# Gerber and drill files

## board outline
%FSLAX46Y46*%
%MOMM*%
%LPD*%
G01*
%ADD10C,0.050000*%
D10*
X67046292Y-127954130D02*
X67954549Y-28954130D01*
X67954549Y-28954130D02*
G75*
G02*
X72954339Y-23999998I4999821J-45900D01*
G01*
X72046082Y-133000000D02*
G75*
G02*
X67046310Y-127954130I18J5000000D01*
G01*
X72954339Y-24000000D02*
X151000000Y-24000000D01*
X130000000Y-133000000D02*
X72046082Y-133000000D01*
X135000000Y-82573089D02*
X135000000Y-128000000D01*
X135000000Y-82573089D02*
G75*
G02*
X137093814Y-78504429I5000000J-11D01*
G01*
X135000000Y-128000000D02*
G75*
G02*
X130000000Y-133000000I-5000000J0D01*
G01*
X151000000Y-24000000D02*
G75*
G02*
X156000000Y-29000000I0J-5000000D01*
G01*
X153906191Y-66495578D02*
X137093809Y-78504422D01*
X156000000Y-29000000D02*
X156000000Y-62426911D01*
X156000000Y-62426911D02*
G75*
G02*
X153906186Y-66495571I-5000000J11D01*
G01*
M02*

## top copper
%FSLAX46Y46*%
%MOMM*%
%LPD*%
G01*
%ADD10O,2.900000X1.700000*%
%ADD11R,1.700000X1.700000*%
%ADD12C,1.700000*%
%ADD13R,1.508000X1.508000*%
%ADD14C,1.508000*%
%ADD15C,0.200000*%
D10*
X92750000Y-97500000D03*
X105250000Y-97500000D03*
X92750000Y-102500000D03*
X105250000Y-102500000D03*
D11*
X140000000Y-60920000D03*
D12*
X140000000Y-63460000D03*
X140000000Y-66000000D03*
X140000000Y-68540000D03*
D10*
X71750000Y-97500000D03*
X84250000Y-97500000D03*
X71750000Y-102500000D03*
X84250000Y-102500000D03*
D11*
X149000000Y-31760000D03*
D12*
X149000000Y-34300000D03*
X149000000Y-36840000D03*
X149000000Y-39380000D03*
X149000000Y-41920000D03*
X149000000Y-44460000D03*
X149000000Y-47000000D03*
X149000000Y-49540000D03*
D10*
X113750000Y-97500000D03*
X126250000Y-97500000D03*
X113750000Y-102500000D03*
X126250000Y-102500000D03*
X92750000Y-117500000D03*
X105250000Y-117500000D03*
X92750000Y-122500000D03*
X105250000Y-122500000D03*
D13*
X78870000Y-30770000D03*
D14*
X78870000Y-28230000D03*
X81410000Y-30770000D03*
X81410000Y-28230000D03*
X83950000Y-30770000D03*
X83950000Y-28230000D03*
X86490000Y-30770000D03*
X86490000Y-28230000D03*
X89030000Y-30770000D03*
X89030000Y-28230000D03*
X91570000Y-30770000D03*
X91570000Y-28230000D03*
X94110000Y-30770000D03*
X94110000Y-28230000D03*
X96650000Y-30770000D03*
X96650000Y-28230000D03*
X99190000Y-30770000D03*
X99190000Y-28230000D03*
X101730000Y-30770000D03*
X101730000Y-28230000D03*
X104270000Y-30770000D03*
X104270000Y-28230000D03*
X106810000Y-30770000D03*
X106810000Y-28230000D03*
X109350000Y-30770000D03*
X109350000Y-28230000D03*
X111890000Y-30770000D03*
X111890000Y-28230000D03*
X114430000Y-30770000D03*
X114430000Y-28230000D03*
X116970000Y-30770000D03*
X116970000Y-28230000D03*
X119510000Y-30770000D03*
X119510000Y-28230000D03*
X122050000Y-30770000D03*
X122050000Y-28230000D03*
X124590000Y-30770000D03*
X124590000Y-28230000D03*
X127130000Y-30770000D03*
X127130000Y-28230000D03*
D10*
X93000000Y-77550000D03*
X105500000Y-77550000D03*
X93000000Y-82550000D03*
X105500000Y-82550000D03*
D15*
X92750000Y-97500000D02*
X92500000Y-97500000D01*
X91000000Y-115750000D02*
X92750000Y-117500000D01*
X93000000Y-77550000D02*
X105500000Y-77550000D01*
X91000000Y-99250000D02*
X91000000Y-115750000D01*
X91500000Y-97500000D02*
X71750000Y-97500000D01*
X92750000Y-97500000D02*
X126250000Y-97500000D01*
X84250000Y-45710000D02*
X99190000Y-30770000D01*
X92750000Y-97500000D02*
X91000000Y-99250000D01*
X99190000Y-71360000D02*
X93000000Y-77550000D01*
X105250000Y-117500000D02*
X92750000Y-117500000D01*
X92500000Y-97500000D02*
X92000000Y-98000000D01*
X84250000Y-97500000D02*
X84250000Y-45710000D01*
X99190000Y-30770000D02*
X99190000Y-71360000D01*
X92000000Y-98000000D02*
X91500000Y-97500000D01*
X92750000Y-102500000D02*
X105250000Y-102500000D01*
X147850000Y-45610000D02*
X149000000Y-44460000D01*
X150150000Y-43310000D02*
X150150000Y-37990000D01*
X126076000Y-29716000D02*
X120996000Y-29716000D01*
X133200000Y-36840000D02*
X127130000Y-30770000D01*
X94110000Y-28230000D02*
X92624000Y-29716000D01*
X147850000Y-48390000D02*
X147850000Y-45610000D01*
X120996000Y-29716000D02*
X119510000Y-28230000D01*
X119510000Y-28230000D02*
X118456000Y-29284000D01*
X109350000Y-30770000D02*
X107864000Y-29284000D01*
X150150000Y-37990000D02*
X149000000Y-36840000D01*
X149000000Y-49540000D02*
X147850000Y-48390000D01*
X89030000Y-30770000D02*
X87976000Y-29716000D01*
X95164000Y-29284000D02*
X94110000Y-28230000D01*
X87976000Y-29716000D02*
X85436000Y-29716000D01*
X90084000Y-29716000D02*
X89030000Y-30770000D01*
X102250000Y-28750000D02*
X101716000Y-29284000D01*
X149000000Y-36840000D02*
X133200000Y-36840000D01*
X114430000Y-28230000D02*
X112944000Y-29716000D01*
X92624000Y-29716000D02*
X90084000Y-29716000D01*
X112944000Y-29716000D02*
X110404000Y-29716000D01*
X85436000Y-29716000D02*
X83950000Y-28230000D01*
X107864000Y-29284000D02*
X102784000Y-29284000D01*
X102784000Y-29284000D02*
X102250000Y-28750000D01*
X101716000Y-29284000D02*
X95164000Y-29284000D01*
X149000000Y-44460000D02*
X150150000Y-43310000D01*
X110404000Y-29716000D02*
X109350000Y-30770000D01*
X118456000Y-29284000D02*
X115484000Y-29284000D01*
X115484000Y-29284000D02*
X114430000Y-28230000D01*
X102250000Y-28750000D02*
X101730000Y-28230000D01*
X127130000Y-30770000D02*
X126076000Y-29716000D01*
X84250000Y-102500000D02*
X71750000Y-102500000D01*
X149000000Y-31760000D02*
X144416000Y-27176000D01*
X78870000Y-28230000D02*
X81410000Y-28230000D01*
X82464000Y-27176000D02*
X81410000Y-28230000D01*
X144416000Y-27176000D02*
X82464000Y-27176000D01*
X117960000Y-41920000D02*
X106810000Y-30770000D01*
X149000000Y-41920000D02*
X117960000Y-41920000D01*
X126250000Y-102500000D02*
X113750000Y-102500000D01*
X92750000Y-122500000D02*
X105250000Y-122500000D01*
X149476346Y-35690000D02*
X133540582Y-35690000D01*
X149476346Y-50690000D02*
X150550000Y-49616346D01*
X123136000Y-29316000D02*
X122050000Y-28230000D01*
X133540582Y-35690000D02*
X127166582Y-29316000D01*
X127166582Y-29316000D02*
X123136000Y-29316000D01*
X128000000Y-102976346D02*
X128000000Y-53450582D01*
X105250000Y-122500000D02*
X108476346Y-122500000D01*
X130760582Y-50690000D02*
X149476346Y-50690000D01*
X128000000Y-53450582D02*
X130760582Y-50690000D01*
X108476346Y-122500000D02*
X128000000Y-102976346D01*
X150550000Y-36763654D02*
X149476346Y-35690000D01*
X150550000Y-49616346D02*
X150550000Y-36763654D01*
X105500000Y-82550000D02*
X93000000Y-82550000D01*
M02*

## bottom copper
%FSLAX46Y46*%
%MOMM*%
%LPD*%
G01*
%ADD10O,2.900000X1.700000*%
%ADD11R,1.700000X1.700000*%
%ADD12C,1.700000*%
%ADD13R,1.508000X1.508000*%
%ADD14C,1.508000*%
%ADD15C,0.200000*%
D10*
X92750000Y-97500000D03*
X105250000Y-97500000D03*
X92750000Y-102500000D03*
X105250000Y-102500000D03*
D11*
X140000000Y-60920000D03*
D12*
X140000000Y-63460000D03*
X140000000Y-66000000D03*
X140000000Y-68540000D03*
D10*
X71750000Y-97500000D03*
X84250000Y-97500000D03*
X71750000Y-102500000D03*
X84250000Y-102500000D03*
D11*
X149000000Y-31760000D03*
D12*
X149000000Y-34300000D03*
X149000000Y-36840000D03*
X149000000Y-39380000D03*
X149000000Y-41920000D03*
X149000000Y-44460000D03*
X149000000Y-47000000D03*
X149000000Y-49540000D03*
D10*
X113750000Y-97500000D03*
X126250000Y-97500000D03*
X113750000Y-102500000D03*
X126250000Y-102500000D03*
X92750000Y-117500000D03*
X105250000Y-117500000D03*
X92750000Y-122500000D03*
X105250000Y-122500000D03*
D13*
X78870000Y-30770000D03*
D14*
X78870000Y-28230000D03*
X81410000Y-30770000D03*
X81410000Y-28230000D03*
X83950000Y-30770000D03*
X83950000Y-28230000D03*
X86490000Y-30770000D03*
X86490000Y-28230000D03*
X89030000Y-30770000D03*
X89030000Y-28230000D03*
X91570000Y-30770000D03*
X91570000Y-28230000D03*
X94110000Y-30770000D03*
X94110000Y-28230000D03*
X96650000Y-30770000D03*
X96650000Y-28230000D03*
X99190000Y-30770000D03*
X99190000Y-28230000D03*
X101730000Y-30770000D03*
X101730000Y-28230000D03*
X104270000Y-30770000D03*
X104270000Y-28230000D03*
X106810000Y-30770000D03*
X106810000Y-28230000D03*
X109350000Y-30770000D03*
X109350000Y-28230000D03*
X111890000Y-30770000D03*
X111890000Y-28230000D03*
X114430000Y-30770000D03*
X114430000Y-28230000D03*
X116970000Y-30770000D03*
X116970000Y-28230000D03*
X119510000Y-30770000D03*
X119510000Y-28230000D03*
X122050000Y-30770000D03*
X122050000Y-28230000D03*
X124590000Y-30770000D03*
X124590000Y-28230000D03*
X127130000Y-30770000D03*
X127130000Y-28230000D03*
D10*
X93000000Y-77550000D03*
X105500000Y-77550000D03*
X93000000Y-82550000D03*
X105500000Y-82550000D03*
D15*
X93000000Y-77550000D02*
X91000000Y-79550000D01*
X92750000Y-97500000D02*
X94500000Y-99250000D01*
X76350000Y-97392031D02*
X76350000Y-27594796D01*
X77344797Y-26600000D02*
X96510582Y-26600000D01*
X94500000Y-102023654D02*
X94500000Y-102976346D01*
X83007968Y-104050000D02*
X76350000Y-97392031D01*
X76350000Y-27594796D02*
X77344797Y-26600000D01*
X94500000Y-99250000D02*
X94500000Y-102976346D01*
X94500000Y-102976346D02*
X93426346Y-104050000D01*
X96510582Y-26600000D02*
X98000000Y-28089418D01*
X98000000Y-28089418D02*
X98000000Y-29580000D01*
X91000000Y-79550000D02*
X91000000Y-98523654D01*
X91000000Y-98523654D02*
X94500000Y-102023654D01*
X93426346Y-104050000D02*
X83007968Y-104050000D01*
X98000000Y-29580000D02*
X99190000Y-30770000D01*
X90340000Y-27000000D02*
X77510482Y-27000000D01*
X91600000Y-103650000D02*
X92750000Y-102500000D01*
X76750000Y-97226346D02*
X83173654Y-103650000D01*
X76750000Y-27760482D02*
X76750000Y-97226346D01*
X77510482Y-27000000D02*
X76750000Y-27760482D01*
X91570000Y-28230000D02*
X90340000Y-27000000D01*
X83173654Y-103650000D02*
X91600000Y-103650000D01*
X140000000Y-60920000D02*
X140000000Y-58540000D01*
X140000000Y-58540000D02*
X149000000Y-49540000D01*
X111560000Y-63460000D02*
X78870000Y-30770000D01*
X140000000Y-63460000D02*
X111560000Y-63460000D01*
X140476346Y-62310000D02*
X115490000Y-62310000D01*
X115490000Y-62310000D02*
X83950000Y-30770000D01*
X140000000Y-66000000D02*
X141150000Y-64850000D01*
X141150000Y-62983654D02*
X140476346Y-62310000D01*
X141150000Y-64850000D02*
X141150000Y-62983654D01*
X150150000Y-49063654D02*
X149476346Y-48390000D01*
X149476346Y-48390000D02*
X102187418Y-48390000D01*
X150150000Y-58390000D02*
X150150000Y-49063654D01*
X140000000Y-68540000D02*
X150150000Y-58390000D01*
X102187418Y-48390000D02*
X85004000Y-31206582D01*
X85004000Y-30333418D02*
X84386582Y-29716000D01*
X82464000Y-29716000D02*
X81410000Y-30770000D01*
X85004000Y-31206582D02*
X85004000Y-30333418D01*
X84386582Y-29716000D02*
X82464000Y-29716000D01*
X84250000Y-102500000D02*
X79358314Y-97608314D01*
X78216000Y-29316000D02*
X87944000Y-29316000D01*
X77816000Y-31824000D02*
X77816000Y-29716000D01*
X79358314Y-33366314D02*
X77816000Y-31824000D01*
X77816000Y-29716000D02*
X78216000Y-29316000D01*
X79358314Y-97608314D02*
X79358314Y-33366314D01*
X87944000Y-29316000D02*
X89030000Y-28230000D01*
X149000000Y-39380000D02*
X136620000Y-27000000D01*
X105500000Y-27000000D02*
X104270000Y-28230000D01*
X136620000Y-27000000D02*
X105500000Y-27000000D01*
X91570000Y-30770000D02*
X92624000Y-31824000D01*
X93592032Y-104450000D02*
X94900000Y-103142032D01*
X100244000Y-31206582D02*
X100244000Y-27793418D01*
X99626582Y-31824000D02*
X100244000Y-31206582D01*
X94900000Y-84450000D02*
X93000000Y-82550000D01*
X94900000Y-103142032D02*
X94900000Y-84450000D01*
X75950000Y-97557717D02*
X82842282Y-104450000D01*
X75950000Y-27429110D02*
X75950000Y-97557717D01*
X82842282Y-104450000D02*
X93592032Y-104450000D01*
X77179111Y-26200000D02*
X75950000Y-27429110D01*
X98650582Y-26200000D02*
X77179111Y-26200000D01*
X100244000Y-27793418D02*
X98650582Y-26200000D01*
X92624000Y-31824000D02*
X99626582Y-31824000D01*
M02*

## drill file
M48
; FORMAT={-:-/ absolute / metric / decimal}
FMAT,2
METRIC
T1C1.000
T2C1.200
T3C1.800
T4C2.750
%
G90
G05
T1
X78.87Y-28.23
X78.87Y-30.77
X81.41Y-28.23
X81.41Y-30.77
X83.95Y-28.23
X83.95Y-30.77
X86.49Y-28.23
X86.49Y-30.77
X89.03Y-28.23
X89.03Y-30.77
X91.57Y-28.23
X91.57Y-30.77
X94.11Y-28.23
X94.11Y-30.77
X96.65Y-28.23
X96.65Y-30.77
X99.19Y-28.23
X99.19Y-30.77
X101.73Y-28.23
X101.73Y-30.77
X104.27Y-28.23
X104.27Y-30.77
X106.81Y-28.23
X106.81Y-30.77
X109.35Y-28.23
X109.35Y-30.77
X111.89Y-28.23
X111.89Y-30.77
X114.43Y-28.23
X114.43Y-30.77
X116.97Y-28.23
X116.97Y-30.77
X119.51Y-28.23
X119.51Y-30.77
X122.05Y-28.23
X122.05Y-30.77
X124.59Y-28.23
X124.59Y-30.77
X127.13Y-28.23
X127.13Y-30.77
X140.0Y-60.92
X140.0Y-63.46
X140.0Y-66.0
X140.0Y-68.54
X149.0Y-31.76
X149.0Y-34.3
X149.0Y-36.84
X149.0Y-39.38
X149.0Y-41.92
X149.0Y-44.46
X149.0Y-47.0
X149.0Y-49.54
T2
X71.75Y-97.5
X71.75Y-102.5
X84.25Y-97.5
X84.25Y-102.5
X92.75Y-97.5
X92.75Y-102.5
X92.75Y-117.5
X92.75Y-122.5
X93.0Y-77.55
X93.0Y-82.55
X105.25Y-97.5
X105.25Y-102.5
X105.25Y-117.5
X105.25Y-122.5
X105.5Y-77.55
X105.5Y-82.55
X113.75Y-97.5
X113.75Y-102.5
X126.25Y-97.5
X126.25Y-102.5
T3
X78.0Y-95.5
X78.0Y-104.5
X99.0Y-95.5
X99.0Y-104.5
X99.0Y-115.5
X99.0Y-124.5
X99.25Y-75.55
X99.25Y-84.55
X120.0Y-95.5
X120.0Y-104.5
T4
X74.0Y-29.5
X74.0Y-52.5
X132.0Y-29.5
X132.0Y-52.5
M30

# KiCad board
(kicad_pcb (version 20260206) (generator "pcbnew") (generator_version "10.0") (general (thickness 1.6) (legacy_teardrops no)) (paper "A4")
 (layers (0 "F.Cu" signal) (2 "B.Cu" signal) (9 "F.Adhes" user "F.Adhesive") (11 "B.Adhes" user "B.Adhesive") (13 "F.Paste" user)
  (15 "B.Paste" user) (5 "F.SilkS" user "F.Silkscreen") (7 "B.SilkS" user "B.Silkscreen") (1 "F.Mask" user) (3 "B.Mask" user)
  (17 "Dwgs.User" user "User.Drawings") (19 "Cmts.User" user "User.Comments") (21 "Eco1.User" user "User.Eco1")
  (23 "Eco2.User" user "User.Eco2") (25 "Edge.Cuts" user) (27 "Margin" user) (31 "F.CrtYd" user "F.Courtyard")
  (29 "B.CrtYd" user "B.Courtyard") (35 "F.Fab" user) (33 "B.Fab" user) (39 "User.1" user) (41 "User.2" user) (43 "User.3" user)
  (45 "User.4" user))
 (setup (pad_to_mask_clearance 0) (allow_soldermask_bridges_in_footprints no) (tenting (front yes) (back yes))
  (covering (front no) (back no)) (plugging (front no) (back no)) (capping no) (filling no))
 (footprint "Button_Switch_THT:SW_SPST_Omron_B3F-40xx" (layer "F.Cu") (at 92.75 97.5)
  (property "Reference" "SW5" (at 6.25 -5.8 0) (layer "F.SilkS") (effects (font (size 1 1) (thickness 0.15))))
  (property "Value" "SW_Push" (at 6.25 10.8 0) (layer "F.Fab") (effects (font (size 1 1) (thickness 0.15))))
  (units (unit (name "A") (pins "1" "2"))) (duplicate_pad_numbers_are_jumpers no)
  (pad "" np_thru_hole circle (at 6.25 -2) (size 1.8 1.8) (drill 1.8) (layers "*.Cu" "*.Mask"))
  (pad "" np_thru_hole circle (at 6.25 7) (size 1.8 1.8) (drill 1.8) (layers "*.Cu" "*.Mask"))
  (pad "1" thru_hole oval (at 0 0) (size 2.9 1.7) (drill 1.2) (layers "*.Cu" "*.Mask") (remove_unused_layers no) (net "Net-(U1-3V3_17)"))
  (pad "1" thru_hole oval (at 12.5 0) (size 2.9 1.7) (drill 1.2) (layers "*.Cu" "*.Mask") (remove_unused_layers no) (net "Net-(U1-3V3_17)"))
  (pad "2" thru_hole oval (at 0 5) (size 2.9 1.7) (drill 1.2) (layers "*.Cu" "*.Mask") (remove_unused_layers no)
   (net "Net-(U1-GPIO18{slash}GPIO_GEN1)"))
  (pad "2" thru_hole oval (at 12.5 5) (size 2.9 1.7) (drill 1.2) (layers "*.Cu" "*.Mask") (remove_unused_layers no)
   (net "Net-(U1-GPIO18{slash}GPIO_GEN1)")))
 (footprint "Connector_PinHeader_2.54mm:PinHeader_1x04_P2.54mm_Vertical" (layer "F.Cu") (at 140 60.92)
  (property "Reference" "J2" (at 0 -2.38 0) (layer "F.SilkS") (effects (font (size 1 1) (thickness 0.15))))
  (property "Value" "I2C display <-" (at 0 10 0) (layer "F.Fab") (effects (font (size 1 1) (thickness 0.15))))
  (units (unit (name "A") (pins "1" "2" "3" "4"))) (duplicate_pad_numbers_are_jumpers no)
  (pad "1" thru_hole rect (at 0 0) (size 1.7 1.7) (drill 1) (layers "*.Cu" "*.Mask") (remove_unused_layers no) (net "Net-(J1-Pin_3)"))
  (pad "2" thru_hole circle (at 0 2.54) (size 1.7 1.7) (drill 1) (layers "*.Cu" "*.Mask") (remove_unused_layers no) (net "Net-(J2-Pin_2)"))
  (pad "3" thru_hole circle (at 0 5.08) (size 1.7 1.7) (drill 1) (layers "*.Cu" "*.Mask") (remove_unused_layers no) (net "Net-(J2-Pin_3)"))
  (pad "4" thru_hole circle (at 0 7.62) (size 1.7 1.7) (drill 1) (layers "*.Cu" "*.Mask") (remove_unused_layers no) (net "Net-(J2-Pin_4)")))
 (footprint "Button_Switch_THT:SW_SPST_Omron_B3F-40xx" (layer "F.Cu") (at 71.75 97.5)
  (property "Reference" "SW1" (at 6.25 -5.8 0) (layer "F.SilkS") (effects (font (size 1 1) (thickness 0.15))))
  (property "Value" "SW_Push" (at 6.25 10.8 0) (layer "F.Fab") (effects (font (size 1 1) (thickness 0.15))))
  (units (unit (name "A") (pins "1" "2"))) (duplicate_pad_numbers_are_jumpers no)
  (pad "" np_thru_hole circle (at 6.25 -2) (size 1.8 1.8) (drill 1.8) (layers "*.Cu" "*.Mask"))
  (pad "" np_thru_hole circle (at 6.25 7) (size 1.8 1.8) (drill 1.8) (layers "*.Cu" "*.Mask"))
  (pad "1" thru_hole oval (at 0 0) (size 2.9 1.7) (drill 1.2) (layers "*.Cu" "*.Mask") (remove_unused_layers no) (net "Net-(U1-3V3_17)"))
  (pad "1" thru_hole oval (at 12.5 0) (size 2.9 1.7) (drill 1.2) (layers "*.Cu" "*.Mask") (remove_unused_layers no) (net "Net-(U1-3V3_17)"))
  (pad "2" thru_hole oval (at 0 5) (size 2.9 1.7) (drill 1.2) (layers "*.Cu" "*.Mask") (remove_unused_layers no)
   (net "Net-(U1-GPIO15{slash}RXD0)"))
  (pad "2" thru_hole oval (at 12.5 5) (size 2.9 1.7) (drill 1.2) (layers "*.Cu" "*.Mask") (remove_unused_layers no)
   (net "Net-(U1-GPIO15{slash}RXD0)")))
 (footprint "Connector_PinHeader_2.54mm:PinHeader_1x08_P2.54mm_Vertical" (layer "F.Cu") (at 149 31.76)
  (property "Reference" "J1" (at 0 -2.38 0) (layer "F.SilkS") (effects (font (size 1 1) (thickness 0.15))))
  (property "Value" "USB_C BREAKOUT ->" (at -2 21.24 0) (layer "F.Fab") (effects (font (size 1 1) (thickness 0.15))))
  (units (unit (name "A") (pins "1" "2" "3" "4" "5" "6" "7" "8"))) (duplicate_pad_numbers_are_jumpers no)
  (pad "1" thru_hole rect (at 0 0) (size 1.7 1.7) (drill 1) (layers "*.Cu" "*.Mask") (remove_unused_layers no) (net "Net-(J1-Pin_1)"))
  (pad "2" thru_hole circle (at 0 2.54) (size 1.7 1.7) (drill 1) (layers "*.Cu" "*.Mask") (remove_unused_layers no)
   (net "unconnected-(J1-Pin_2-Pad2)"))
  (pad "3" thru_hole circle (at 0 5.08) (size 1.7 1.7) (drill 1) (layers "*.Cu" "*.Mask") (remove_unused_layers no) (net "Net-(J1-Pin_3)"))
  (pad "4" thru_hole circle (at 0 7.62) (size 1.7 1.7) (drill 1) (layers "*.Cu" "*.Mask") (remove_unused_layers no) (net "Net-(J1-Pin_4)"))
  (pad "5" thru_hole circle (at 0 10.16) (size 1.7 1.7) (drill 1) (layers "*.Cu" "*.Mask") (remove_unused_layers no) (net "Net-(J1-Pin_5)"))
  (pad "6" thru_hole circle (at 0 12.7) (size 1.7 1.7) (drill 1) (layers "*.Cu" "*.Mask") (remove_unused_layers no) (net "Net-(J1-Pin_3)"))
  (pad "7" thru_hole circle (at 0 15.24) (size 1.7 1.7) (drill 1) (layers "*.Cu" "*.Mask") (remove_unused_layers no)
   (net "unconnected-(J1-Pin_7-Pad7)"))
  (pad "8" thru_hole circle (at 0 17.78) (size 1.7 1.7) (drill 1) (layers "*.Cu" "*.Mask") (remove_unused_layers no) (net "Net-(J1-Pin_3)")))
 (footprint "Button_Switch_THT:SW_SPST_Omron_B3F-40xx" (layer "F.Cu") (at 113.75 97.5)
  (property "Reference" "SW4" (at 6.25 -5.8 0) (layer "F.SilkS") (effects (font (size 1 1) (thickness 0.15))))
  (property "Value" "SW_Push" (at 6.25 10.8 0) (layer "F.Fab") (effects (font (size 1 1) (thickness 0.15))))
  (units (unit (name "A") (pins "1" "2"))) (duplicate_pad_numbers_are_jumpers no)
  (pad "" np_thru_hole circle (at 6.25 -2) (size 1.8 1.8) (drill 1.8) (layers "*.Cu" "*.Mask"))
  (pad "" np_thru_hole circle (at 6.25 7) (size 1.8 1.8) (drill 1.8) (layers "*.Cu" "*.Mask"))
  (pad "1" thru_hole oval (at 0 0) (size 2.9 1.7) (drill 1.2) (layers "*.Cu" "*.Mask") (remove_unused_layers no) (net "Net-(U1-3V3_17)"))
  (pad "1" thru_hole oval (at 12.5 0) (size 2.9 1.7) (drill 1.2) (layers "*.Cu" "*.Mask") (remove_unused_layers no) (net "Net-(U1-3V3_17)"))
  (pad "2" thru_hole oval (at 0 5) (size 2.9 1.7) (drill 1.2) (layers "*.Cu" "*.Mask") (remove_unused_layers no)
   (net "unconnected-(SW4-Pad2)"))
  (pad "2" thru_hole oval (at 12.5 5) (size 2.9 1.7) (drill 1.2) (layers "*.Cu" "*.Mask") (remove_unused_layers no)
   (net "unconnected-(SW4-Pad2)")))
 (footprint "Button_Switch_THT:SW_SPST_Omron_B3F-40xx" (layer "F.Cu") (at 92.75 117.5)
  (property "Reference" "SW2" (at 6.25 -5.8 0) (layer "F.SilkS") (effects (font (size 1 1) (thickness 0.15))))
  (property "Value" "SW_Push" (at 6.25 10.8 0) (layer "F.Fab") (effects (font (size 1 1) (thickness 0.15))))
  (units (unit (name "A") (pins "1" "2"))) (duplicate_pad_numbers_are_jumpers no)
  (pad "" np_thru_hole circle (at 6.25 -2) (size 1.8 1.8) (drill 1.8) (layers "*.Cu" "*.Mask"))
  (pad "" np_thru_hole circle (at 6.25 7) (size 1.8 1.8) (drill 1.8) (layers "*.Cu" "*.Mask"))
  (pad "1" thru_hole oval (at 0 0) (size 2.9 1.7) (drill 1.2) (layers "*.Cu" "*.Mask") (remove_unused_layers no) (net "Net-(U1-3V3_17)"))
  (pad "1" thru_hole oval (at 12.5 0) (size 2.9 1.7) (drill 1.2) (layers "*.Cu" "*.Mask") (remove_unused_layers no) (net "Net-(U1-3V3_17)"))
  (pad "2" thru_hole oval (at 0 5) (size 2.9 1.7) (drill 1.2) (layers "*.Cu" "*.Mask") (remove_unused_layers no) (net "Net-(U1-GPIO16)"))
  (pad "2" thru_hole oval (at 12.5 5) (size 2.9 1.7) (drill 1.2) (layers "*.Cu" "*.Mask") (remove_unused_layers no) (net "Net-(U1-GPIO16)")))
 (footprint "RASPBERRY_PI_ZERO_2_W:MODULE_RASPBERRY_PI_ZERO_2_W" (layer "F.Cu") (at 103 41)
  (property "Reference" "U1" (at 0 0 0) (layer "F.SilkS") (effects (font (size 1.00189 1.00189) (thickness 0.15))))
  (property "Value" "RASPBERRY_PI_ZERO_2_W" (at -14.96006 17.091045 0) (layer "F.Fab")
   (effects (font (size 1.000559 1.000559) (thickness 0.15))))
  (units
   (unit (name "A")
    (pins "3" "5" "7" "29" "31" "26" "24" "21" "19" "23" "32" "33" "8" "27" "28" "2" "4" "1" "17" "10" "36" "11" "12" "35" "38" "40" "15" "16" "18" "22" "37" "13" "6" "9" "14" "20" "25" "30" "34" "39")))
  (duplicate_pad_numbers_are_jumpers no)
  (pad "" np_thru_hole circle (at -29 -11.5) (size 2.75 2.75) (drill 2.75) (layers "*.Cu" "*.Mask"))
  (pad "" np_thru_hole circle (at -29 11.5) (size 2.75 2.75) (drill 2.75) (layers "*.Cu" "*.Mask"))
  (pad "" np_thru_hole circle (at 29 -11.5) (size 2.75 2.75) (drill 2.75) (layers "*.Cu" "*.Mask"))
  (pad "" np_thru_hole circle (at 29 11.5) (size 2.75 2.75) (drill 2.75) (layers "*.Cu" "*.Mask"))
  (pad "1" thru_hole rect (at -24.13 -10.23) (size 1.508 1.508) (drill 1) (layers "*.Cu" "*.Mask") (remove_unused_layers no)
   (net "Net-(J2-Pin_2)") (solder_mask_margin 0.102))
  (pad "2" thru_hole circle (at -24.13 -12.77) (size 1.508 1.508) (drill 1) (layers "*.Cu" "*.Mask") (remove_unused_layers no)
   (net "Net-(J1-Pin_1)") (solder_mask_margin 0.102))
  (pad "3" thru_hole circle (at -21.59 -10.23) (size 1.508 1.508) (drill 1) (layers "*.Cu" "*.Mask") (remove_unused_layers no)
   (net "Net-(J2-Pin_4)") (solder_mask_margin 0.102))
  (pad "4" thru_hole circle (at -21.59 -12.77) (size 1.508 1.508) (drill 1) (layers "*.Cu" "*.Mask") (remove_unused_layers no)
   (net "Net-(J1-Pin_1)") (solder_mask_margin 0.102))
  (pad "5" thru_hole circle (at -19.05 -10.23) (size 1.508 1.508) (drill 1) (layers "*.Cu" "*.Mask") (remove_unused_layers no)
   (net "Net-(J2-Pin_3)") (solder_mask_margin 0.102))
  (pad "6" thru_hole circle (at -19.05 -12.77) (size 1.508 1.508) (drill 1) (layers "*.Cu" "*.Mask") (remove_unused_layers no)
   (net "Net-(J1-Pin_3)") (solder_mask_margin 0.102))
  (pad "7" thru_hole circle (at -16.51 -10.23) (size 1.508 1.508) (drill 1) (layers "*.Cu" "*.Mask") (remove_unused_layers no)
   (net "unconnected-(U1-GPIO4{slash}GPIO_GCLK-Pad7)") (solder_mask_margin 0.102))
  (pad "8" thru_hole circle (at -16.51 -12.77) (size 1.508 1.508) (drill 1) (layers "*.Cu" "*.Mask") (remove_unused_layers no)
   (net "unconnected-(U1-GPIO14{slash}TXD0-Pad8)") (solder_mask_margin 0.102))
  (pad "9" thru_hole circle (at -13.97 -10.23) (size 1.508 1.508) (drill 1) (layers "*.Cu" "*.Mask") (remove_unused_layers no)
   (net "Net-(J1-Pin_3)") (solder_mask_margin 0.102))
  (pad "10" thru_hole circle (at -13.97 -12.77) (size 1.508 1.508) (drill 1) (layers "*.Cu" "*.Mask") (remove_unused_layers no)
   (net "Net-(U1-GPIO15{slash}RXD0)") (solder_mask_margin 0.102))
  (pad "11" thru_hole circle (at -11.43 -10.23) (size 1.508 1.508) (drill 1) (layers "*.Cu" "*.Mask") (remove_unused_layers no)
   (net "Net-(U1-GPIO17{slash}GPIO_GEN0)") (solder_mask_margin 0.102))
  (pad "12" thru_hole circle (at -11.43 -12.77) (size 1.508 1.508) (drill 1) (layers "*.Cu" "*.Mask") (remove_unused_layers no)
   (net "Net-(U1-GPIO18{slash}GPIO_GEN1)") (solder_mask_margin 0.102))
  (pad "13" thru_hole circle (at -8.89 -10.23) (size 1.508 1.508) (drill 1) (layers "*.Cu" "*.Mask") (remove_unused_layers no)
   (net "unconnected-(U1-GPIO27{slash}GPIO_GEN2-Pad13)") (solder_mask_margin 0.102))
  (pad "14" thru_hole circle (at -8.89 -12.77) (size 1.508 1.508) (drill 1) (layers "*.Cu" "*.Mask") (remove_unused_layers no)
   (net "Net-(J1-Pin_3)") (solder_mask_margin 0.102))
  (pad "15" thru_hole circle (at -6.35 -10.23) (size 1.508 1.508) (drill 1) (layers "*.Cu" "*.Mask") (remove_unused_layers no)
   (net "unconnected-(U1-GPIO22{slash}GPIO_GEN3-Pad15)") (solder_mask_margin 0.102))
  (pad "16" thru_hole circle (at -6.35 -12.77) (size 1.508 1.508) (drill 1) (layers "*.Cu" "*.Mask") (remove_unused_layers no)
   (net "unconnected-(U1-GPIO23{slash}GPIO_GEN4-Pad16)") (solder_mask_margin 0.102))
  (pad "17" thru_hole circle (at -3.81 -10.23) (size 1.508 1.508) (drill 1) (layers "*.Cu" "*.Mask") (remove_unused_layers no)
   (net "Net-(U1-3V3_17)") (solder_mask_margin 0.102))
  (pad "18" thru_hole circle (at -3.81 -12.77) (size 1.508 1.508) (drill 1) (layers "*.Cu" "*.Mask") (remove_unused_layers no)
   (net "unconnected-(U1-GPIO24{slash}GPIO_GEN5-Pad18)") (solder_mask_margin 0.102))
  (pad "19" thru_hole circle (at -1.27 -10.23) (size 1.508 1.508) (drill 1) (layers "*.Cu" "*.Mask") (remove_unused_layers no)
   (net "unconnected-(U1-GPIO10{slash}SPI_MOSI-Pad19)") (solder_mask_margin 0.102))
  (pad "20" thru_hole circle (at -1.27 -12.77) (size 1.508 1.508) (drill 1) (layers "*.Cu" "*.Mask") (remove_unused_layers no)
   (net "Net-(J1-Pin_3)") (solder_mask_margin 0.102))
  (pad "21" thru_hole circle (at 1.27 -10.23) (size 1.508 1.508) (drill 1) (layers "*.Cu" "*.Mask") (remove_unused_layers no)
   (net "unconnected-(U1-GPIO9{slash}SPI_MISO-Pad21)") (solder_mask_margin 0.102))
  (pad "22" thru_hole circle (at 1.27 -12.77) (size 1.508 1.508) (drill 1) (layers "*.Cu" "*.Mask") (remove_unused_layers no)
   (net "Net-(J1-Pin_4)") (solder_mask_margin 0.102))
  (pad "23" thru_hole circle (at 3.81 -10.23) (size 1.508 1.508) (drill 1) (layers "*.Cu" "*.Mask") (remove_unused_layers no)
   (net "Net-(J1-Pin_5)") (solder_mask_margin 0.102))
  (pad "24" thru_hole circle (at 3.81 -12.77) (size 1.508 1.508) (drill 1) (layers "*.Cu" "*.Mask") (remove_unused_layers no)
   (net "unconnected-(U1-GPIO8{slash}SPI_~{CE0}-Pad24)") (solder_mask_margin 0.102))
  (pad "25" thru_hole circle (at 6.35 -10.23) (size 1.508 1.508) (drill 1) (layers "*.Cu" "*.Mask") (remove_unused_layers no)
   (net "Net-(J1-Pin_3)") (solder_mask_margin 0.102))
  (pad "26" thru_hole circle (at 6.35 -12.77) (size 1.508 1.508) (drill 1) (layers "*.Cu" "*.Mask") (remove_unused_layers no)
   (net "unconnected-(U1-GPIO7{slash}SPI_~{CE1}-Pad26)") (solder_mask_margin 0.102))
  (pad "27" thru_hole circle (at 8.89 -10.23) (size 1.508 1.508) (drill 1) (layers "*.Cu" "*.Mask") (remove_unused_layers no)
   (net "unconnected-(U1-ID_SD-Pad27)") (solder_mask_margin 0.102))
  (pad "28" thru_hole circle (at 8.89 -12.77) (size 1.508 1.508) (drill 1) (layers "*.Cu" "*.Mask") (remove_unused_layers no)
   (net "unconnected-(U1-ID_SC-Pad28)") (solder_mask_margin 0.102))
  (pad "29" thru_hole circle (at 11.43 -10.23) (size 1.508 1.508) (drill 1) (layers "*.Cu" "*.Mask") (remove_unused_layers no)
   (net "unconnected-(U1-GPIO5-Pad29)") (solder_mask_margin 0.102))
  (pad "30" thru_hole circle (at 11.43 -12.77) (size 1.508 1.508) (drill 1) (layers "*.Cu" "*.Mask") (remove_unused_layers no)
   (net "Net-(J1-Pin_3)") (solder_mask_margin 0.102))
  (pad "31" thru_hole circle (at 13.97 -10.23) (size 1.508 1.508) (drill 1) (layers "*.Cu" "*.Mask") (remove_unused_layers no)
   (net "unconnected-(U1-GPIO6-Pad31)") (solder_mask_margin 0.102))
  (pad "32" thru_hole circle (at 13.97 -12.77) (size 1.508 1.508) (drill 1) (layers "*.Cu" "*.Mask") (remove_unused_layers no)
   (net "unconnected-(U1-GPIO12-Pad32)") (solder_mask_margin 0.102))
  (pad "33" thru_hole circle (at 16.51 -10.23) (size 1.508 1.508) (drill 1) (layers "*.Cu" "*.Mask") (remove_unused_layers no)
   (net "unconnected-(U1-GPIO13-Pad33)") (solder_mask_margin 0.102))
  (pad "34" thru_hole circle (at 16.51 -12.77) (size 1.508 1.508) (drill 1) (layers "*.Cu" "*.Mask") (remove_unused_layers no)
   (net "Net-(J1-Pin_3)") (solder_mask_margin 0.102))
  (pad "35" thru_hole circle (at 19.05 -10.23) (size 1.508 1.508) (drill 1) (layers "*.Cu" "*.Mask") (remove_unused_layers no)
   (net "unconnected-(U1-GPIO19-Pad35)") (solder_mask_margin 0.102))
  (pad "36" thru_hole circle (at 19.05 -12.77) (size 1.508 1.508) (drill 1) (layers "*.Cu" "*.Mask") (remove_unused_layers no)
   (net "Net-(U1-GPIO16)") (solder_mask_margin 0.102))
  (pad "37" thru_hole circle (at 21.59 -10.23) (size 1.508 1.508) (drill 1) (layers "*.Cu" "*.Mask") (remove_unused_layers no)
   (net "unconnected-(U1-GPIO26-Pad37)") (solder_mask_margin 0.102))
  (pad "38" thru_hole circle (at 21.59 -12.77) (size 1.508 1.508) (drill 1) (layers "*.Cu" "*.Mask") (remove_unused_layers no)
   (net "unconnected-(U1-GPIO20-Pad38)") (solder_mask_margin 0.102))
  (pad "39" thru_hole circle (at 24.13 -10.23) (size 1.508 1.508) (drill 1) (layers "*.Cu" "*.Mask") (remove_unused_layers no)
   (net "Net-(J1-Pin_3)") (solder_mask_margin 0.102))
  (pad "40" thru_hole circle (at 24.13 -12.77) (size 1.508 1.508) (drill 1) (layers "*.Cu" "*.Mask") (remove_unused_layers no)
   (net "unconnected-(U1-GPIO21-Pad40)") (solder_mask_margin 0.102)))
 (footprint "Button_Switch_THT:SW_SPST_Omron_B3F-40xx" (layer "F.Cu") (at 93 77.55)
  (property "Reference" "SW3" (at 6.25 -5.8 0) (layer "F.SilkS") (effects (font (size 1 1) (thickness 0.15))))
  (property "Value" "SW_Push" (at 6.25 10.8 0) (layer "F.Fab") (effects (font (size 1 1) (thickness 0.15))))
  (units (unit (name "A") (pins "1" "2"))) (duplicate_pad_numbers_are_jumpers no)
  (pad "" np_thru_hole circle (at 6.25 -2) (size 1.8 1.8) (drill 1.8) (layers "*.Cu" "*.Mask"))
  (pad "" np_thru_hole circle (at 6.25 7) (size 1.8 1.8) (drill 1.8) (layers "*.Cu" "*.Mask"))
  (pad "1" thru_hole oval (at 0 0) (size 2.9 1.7) (drill 1.2) (layers "*.Cu" "*.Mask") (remove_unused_layers no) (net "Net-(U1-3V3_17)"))
  (pad "1" thru_hole oval (at 12.5 0) (size 2.9 1.7) (drill 1.2) (layers "*.Cu" "*.Mask") (remove_unused_layers no) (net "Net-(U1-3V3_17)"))
  (pad "2" thru_hole oval (at 0 5) (size 2.9 1.7) (drill 1.2) (layers "*.Cu" "*.Mask") (remove_unused_layers no)
   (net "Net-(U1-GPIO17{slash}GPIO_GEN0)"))
  (pad "2" thru_hole oval (at 12.5 5) (size 2.9 1.7) (drill 1.2) (layers "*.Cu" "*.Mask") (remove_unused_layers no)
   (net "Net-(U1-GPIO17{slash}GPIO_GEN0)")))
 (gr_line (start 67.046292 127.95413) (end 67.954549 28.95413) (stroke (width 0.05) (type default)) (layer "Edge.Cuts"))
 (gr_arc (start 67.954549 28.95413) (mid 69.435062 25.448299) (end 72.954339 24) (stroke (width 0.05) (type default)) (layer "Edge.Cuts"))
 (gr_arc (start 72.046082 133) (mid 68.494368 131.519279) (end 67.046292 127.95413) (stroke (width 0.05) (type default)) (layer "Edge.Cuts"))
 (gr_line (start 72.954339 24) (end 151 24) (stroke (width 0.05) (type default)) (layer "Edge.Cuts"))
 (gr_line (start 130 133) (end 72.046082 133) (stroke (width 0.05) (type default)) (layer "Edge.Cuts"))
 (gr_line (start 135 82.573089) (end 135 128) (stroke (width 0.05) (type default)) (layer "Edge.Cuts"))
 (gr_arc (start 135 82.573089) (mid 135.554166 80.285184) (end 137.093809 78.504422) (stroke (width 0.05) (type default))
  (layer "Edge.Cuts"))
 (gr_arc (start 135 128) (mid 133.535534 131.535534) (end 130 133) (stroke (width 0.05) (type default)) (layer "Edge.Cuts"))
 (gr_arc (start 151 24) (mid 154.535534 25.464466) (end 156 29) (stroke (width 0.05) (type default)) (layer "Edge.Cuts"))
 (gr_line (start 153.906191 66.495578) (end 137.093809 78.504422) (stroke (width 0.05) (type default)) (layer "Edge.Cuts"))
 (gr_line (start 156 29) (end 156 62.426911) (stroke (width 0.05) (type default)) (layer "Edge.Cuts"))
 (gr_arc (start 156 62.426911) (mid 155.445834 64.714816) (end 153.906191 66.495578) (stroke (width 0.05) (type default))
  (layer "Edge.Cuts"))
 (segment (start 92.75 97.5) (end 92.5 97.5) (width 0.2) (layer "F.Cu") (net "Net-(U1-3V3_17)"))
 (segment (start 91 115.75) (end 92.75 117.5) (width 0.2) (layer "F.Cu") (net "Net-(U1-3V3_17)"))
 (segment (start 93 77.55) (end 105.5 77.55) (width 0.2) (layer "F.Cu") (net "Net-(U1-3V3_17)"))
 (segment (start 91 99.25) (end 91 115.75) (width 0.2) (layer "F.Cu") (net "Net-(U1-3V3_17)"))
 (segment (start 91.5 97.5) (end 71.75 97.5) (width 0.2) (layer "F.Cu") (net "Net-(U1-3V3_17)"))
 (segment (start 92.75 97.5) (end 126.25 97.5) (width 0.2) (layer "F.Cu") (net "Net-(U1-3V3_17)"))
 (segment (start 84.25 45.71) (end 99.19 30.77) (width 0.2) (layer "F.Cu") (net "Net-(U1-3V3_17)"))
 (segment (start 92.75 97.5) (end 91 99.25) (width 0.2) (layer "F.Cu") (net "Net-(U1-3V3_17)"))
 (segment (start 99.19 71.36) (end 93 77.55) (width 0.2) (layer "F.Cu") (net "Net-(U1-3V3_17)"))
 (segment (start 105.25 117.5) (end 92.75 117.5) (width 0.2) (layer "F.Cu") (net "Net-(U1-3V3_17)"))
 (segment (start 92.5 97.5) (end 92 98) (width 0.2) (layer "F.Cu") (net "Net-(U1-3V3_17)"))
 (segment (start 84.25 97.5) (end 84.25 45.71) (width 0.2) (layer "F.Cu") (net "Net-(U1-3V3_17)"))
 (segment (start 99.19 30.77) (end 99.19 71.36) (width 0.2) (layer "F.Cu") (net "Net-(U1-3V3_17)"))
 (segment (start 92 98) (end 91.5 97.5) (width 0.2) (layer "F.Cu") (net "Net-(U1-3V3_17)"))
 (segment (start 93 77.55) (end 91 79.55) (width 0.2) (layer "B.Cu") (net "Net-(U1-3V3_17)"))
 (segment (start 92.75 97.5) (end 94.5 99.25) (width 0.2) (layer "B.Cu") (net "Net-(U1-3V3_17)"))
 (segment (start 76.35 97.392031) (end 76.35 27.594796) (width 0.2) (layer "B.Cu") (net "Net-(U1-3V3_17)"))
 (segment (start 77.344797 26.6) (end 96.510582 26.6) (width 0.2) (layer "B.Cu") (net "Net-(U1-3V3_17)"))
 (segment (start 94.5 102.023654) (end 94.5 102.976346) (width 0.2) (layer "B.Cu") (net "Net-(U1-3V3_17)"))
 (segment (start 83.007968 104.05) (end 76.35 97.392031) (width 0.2) (layer "B.Cu") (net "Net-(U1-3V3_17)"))
 (segment (start 76.35 27.594796) (end 77.344797 26.6) (width 0.2) (layer "B.Cu") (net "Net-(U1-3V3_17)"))
 (segment (start 94.5 99.25) (end 94.5 102.976346) (width 0.2) (layer "B.Cu") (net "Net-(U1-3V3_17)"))
 (segment (start 94.5 102.976346) (end 93.426346 104.05) (width 0.2) (layer "B.Cu") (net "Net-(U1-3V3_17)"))
 (segment (start 96.510582 26.6) (end 98 28.089418) (width 0.2) (layer "B.Cu") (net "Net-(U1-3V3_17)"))
 (segment (start 98 28.089418) (end 98 29.58) (width 0.2) (layer "B.Cu") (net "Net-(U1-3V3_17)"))
 (segment (start 91 79.55) (end 91 98.523654) (width 0.2) (layer "B.Cu") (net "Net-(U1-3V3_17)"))
 (segment (start 91 98.523654) (end 94.5 102.023654) (width 0.2) (layer "B.Cu") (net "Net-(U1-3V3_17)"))
 (segment (start 93.426346 104.05) (end 83.007968 104.05) (width 0.2) (layer "B.Cu") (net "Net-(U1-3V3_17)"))
 (segment (start 98 29.58) (end 99.19 30.77) (width 0.2) (layer "B.Cu") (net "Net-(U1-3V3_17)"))
 (segment (start 92.75 102.5) (end 105.25 102.5) (width 0.2) (layer "F.Cu") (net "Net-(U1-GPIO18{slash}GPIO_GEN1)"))
 (segment (start 90.34 27) (end 77.510482 27) (width 0.2) (layer "B.Cu") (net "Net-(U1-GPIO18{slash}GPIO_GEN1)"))
 (segment (start 91.6 103.65) (end 92.75 102.5) (width 0.2) (layer "B.Cu") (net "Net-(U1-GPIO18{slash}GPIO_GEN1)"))
 (segment (start 76.75 97.226346) (end 83.173654 103.65) (width 0.2) (layer "B.Cu") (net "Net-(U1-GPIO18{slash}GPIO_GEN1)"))
 (segment (start 76.75 27.760482) (end 76.75 97.226346) (width 0.2) (layer "B.Cu") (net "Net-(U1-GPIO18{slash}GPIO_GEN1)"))
 (segment (start 77.510482 27) (end 76.75 27.760482) (width 0.2) (layer "B.Cu") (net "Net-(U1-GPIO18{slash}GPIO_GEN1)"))
 (segment (start 91.57 28.23) (end 90.34 27) (width 0.2) (layer "B.Cu") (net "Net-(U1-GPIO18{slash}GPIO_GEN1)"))
 (segment (start 83.173654 103.65) (end 91.6 103.65) (width 0.2) (layer "B.Cu") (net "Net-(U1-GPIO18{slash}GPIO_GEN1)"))
 (segment (start 147.85 45.61) (end 149 44.46) (width 0.2) (layer "F.Cu") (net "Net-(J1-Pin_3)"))
 (segment (start 150.15 43.31) (end 150.15 37.99) (width 0.2) (layer "F.Cu") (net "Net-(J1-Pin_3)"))
 (segment (start 126.076 29.716) (end 120.996 29.716) (width 0.2) (layer "F.Cu") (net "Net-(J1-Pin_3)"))
 (segment (start 133.2 36.84) (end 127.13 30.77) (width 0.2) (layer "F.Cu") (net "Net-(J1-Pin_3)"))
 (segment (start 94.11 28.23) (end 92.624 29.716) (width 0.2) (layer "F.Cu") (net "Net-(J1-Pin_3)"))
 (segment (start 147.85 48.39) (end 147.85 45.61) (width 0.2) (layer "F.Cu") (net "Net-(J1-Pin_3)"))
 (segment (start 120.996 29.716) (end 119.51 28.23) (width 0.2) (layer "F.Cu") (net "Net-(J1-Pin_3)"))
 (segment (start 119.51 28.23) (end 118.456 29.284) (width 0.2) (layer "F.Cu") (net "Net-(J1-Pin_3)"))
 (segment (start 109.35 30.77) (end 107.864 29.284) (width 0.2) (layer "F.Cu") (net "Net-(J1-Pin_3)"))
 (segment (start 150.15 37.99) (end 149 36.84) (width 0.2) (layer "F.Cu") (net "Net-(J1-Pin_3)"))
 (segment (start 149 49.54) (end 147.85 48.39) (width 0.2) (layer "F.Cu") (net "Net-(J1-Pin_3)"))
 (segment (start 89.03 30.77) (end 87.976 29.716) (width 0.2) (layer "F.Cu") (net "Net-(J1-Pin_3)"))
 (segment (start 95.164 29.284) (end 94.11 28.23) (width 0.2) (layer "F.Cu") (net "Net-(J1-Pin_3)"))
 (segment (start 87.976 29.716) (end 85.436 29.716) (width 0.2) (layer "F.Cu") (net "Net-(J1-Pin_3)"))
 (segment (start 90.084 29.716) (end 89.03 30.77) (width 0.2) (layer "F.Cu") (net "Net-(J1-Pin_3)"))
 (segment (start 102.25 28.75) (end 101.716 29.284) (width 0.2) (layer "F.Cu") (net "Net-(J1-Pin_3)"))
 (segment (start 149 36.84) (end 133.2 36.84) (width 0.2) (layer "F.Cu") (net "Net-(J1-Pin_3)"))
 (segment (start 114.43 28.23) (end 112.944 29.716) (width 0.2) (layer "F.Cu") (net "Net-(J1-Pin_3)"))
 (segment (start 92.624 29.716) (end 90.084 29.716) (width 0.2) (layer "F.Cu") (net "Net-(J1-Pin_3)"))
 (segment (start 112.944 29.716) (end 110.404 29.716) (width 0.2) (layer "F.Cu") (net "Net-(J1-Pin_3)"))
 (segment (start 85.436 29.716) (end 83.95 28.23) (width 0.2) (layer "F.Cu") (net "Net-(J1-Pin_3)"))
 (segment (start 107.864 29.284) (end 102.784 29.284) (width 0.2) (layer "F.Cu") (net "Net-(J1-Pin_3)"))
 (segment (start 102.784 29.284) (end 102.25 28.75) (width 0.2) (layer "F.Cu") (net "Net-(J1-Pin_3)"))
 (segment (start 101.716 29.284) (end 95.164 29.284) (width 0.2) (layer "F.Cu") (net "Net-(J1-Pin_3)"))
 (segment (start 149 44.46) (end 150.15 43.31) (width 0.2) (layer "F.Cu") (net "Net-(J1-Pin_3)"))
 (segment (start 110.404 29.716) (end 109.35 30.77) (width 0.2) (layer "F.Cu") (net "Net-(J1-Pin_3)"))
 (segment (start 118.456 29.284) (end 115.484 29.284) (width 0.2) (layer "F.Cu") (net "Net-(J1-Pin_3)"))
 (segment (start 115.484 29.284) (end 114.43 28.23) (width 0.2) (layer "F.Cu") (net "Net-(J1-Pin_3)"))
 (segment (start 102.25 28.75) (end 101.73 28.23) (width 0.2) (layer "F.Cu") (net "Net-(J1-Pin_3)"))
 (segment (start 127.13 30.77) (end 126.076 29.716) (width 0.2) (layer "F.Cu") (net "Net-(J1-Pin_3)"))
 (segment (start 140 60.92) (end 140 58.54) (width 0.2) (layer "B.Cu") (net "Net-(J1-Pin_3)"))
 (segment (start 140 58.54) (end 149 49.54) (width 0.2) (layer "B.Cu") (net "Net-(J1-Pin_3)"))
 (segment (start 111.56 63.46) (end 78.87 30.77) (width 0.2) (layer "B.Cu") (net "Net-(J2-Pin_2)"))
 (segment (start 140 63.46) (end 111.56 63.46) (width 0.2) (layer "B.Cu") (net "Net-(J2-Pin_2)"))
 (segment (start 140.476346 62.31) (end 115.49 62.31) (width 0.2) (layer "B.Cu") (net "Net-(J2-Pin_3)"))
 (segment (start 115.49 62.31) (end 83.95 30.77) (width 0.2) (layer "B.Cu") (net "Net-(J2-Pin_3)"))
 (segment (start 140 66) (end 141.15 64.85) (width 0.2) (layer "B.Cu") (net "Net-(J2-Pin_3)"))
 (segment (start 141.15 62.983654) (end 140.476346 62.31) (width 0.2) (layer "B.Cu") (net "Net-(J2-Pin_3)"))
 (segment (start 141.15 64.85) (end 141.15 62.983654) (width 0.2) (layer "B.Cu") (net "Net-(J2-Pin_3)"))
 (segment (start 150.15 49.063654) (end 149.476346 48.39) (width 0.2) (layer "B.Cu") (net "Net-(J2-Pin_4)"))
 (segment (start 149.476346 48.39) (end 102.187418 48.39) (width 0.2) (layer "B.Cu") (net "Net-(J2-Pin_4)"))
 (segment (start 150.15 58.39) (end 150.15 49.063654) (width 0.2) (layer "B.Cu") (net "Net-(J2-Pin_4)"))
 (segment (start 140 68.54) (end 150.15 58.39) (width 0.2) (layer "B.Cu") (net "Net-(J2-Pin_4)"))
 (segment (start 102.187418 48.39) (end 85.004 31.206582) (width 0.2) (layer "B.Cu") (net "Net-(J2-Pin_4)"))
 (segment (start 85.004 30.333418) (end 84.386582 29.716) (width 0.2) (layer "B.Cu") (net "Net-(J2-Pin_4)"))
 (segment (start 82.464 29.716) (end 81.41 30.77) (width 0.2) (layer "B.Cu") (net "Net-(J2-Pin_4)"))
 (segment (start 85.004 31.206582) (end 85.004 30.333418) (width 0.2) (layer "B.Cu") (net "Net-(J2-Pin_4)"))
 (segment (start 84.386582 29.716) (end 82.464 29.716) (width 0.2) (layer "B.Cu") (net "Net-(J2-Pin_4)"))
 (segment (start 84.25 102.5) (end 71.75 102.5) (width 0.2) (layer "F.Cu") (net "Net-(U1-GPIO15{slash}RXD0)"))
 (segment (start 84.25 102.5) (end 79.358314 97.608314) (width 0.2) (layer "B.Cu") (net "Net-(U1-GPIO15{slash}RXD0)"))
 (segment (start 78.216 29.316) (end 87.944 29.316) (width 0.2) (layer "B.Cu") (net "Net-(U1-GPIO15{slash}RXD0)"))
 (segment (start 77.816 31.824) (end 77.816 29.716) (width 0.2) (layer "B.Cu") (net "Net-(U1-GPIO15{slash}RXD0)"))
 (segment (start 79.358314 33.366314) (end 77.816 31.824) (width 0.2) (layer "B.Cu") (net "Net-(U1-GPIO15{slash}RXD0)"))
 (segment (start 77.816 29.716) (end 78.216 29.316) (width 0.2) (layer "B.Cu") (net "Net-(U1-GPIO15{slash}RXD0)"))
 (segment (start 79.358314 97.608314) (end 79.358314 33.366314) (width 0.2) (layer "B.Cu") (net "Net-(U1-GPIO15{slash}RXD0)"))
 (segment (start 87.944 29.316) (end 89.03 28.23) (width 0.2) (layer "B.Cu") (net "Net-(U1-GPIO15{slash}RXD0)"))
 (segment (start 149 31.76) (end 144.416 27.176) (width 0.2) (layer "F.Cu") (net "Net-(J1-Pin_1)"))
 (segment (start 78.87 28.23) (end 81.41 28.23) (width 0.2) (layer "F.Cu") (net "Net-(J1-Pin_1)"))
 (segment (start 82.464 27.176) (end 81.41 28.23) (width 0.2) (layer "F.Cu") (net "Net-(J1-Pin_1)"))
 (segment (start 144.416 27.176) (end 82.464 27.176) (width 0.2) (layer "F.Cu") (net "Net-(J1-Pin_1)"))
 (segment (start 149 39.38) (end 136.62 27) (width 0.2) (layer "B.Cu") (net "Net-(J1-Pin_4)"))
 (segment (start 105.5 27) (end 104.27 28.23) (width 0.2) (layer "B.Cu") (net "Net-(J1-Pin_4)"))
 (segment (start 136.62 27) (end 105.5 27) (width 0.2) (layer "B.Cu") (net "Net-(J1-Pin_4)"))
 (segment (start 117.96 41.92) (end 106.81 30.77) (width 0.2) (layer "F.Cu") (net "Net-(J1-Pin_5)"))
 (segment (start 149 41.92) (end 117.96 41.92) (width 0.2) (layer "F.Cu") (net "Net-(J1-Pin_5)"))
 (segment (start 126.25 102.5) (end 113.75 102.5) (width 0.2) (layer "F.Cu") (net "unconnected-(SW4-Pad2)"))
 (segment (start 92.75 122.5) (end 105.25 122.5) (width 0.2) (layer "F.Cu") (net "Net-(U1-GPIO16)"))
 (segment (start 149.476346 35.69) (end 133.540582 35.69) (width 0.2) (layer "F.Cu") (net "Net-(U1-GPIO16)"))
 (segment (start 149.476346 50.69) (end 150.55 49.616346) (width 0.2) (layer "F.Cu") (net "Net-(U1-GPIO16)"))
 (segment (start 123.136 29.316) (end 122.05 28.23) (width 0.2) (layer "F.Cu") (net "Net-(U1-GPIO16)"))
 (segment (start 133.540582 35.69) (end 127.166582 29.316) (width 0.2) (layer "F.Cu") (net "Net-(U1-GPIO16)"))
 (segment (start 127.166582 29.316) (end 123.136 29.316) (width 0.2) (layer "F.Cu") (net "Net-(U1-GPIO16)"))
 (segment (start 128 102.976346) (end 128 53.450582) (width 0.2) (layer "F.Cu") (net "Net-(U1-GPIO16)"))
 (segment (start 105.25 122.5) (end 108.476346 122.5) (width 0.2) (layer "F.Cu") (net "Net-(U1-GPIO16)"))
 (segment (start 130.760582 50.69) (end 149.476346 50.69) (width 0.2) (layer "F.Cu") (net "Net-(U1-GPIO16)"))
 (segment (start 128 53.450582) (end 130.760582 50.69) (width 0.2) (layer "F.Cu") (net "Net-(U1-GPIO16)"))
 (segment (start 108.476346 122.5) (end 128 102.976346) (width 0.2) (layer "F.Cu") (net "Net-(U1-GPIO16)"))
 (segment (start 150.55 36.763654) (end 149.476346 35.69) (width 0.2) (layer "F.Cu") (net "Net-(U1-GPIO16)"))
 (segment (start 150.55 49.616346) (end 150.55 36.763654) (width 0.2) (layer "F.Cu") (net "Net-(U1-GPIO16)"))
 (segment (start 105.5 82.55) (end 93 82.55) (width 0.2) (layer "F.Cu") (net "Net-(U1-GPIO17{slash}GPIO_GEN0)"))
 (segment (start 91.57 30.77) (end 92.624 31.824) (width 0.2) (layer "B.Cu") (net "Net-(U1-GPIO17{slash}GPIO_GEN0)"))
 (segment (start 93.592032 104.45) (end 94.9 103.142032) (width 0.2) (layer "B.Cu") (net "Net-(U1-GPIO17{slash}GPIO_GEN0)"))
 (segment (start 100.244 31.206582) (end 100.244 27.793418) (width 0.2) (layer "B.Cu") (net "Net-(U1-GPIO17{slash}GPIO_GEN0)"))
 (segment (start 99.626582 31.824) (end 100.244 31.206582) (width 0.2) (layer "B.Cu") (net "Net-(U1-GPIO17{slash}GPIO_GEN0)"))
 (segment (start 94.9 84.45) (end 93 82.55) (width 0.2) (layer "B.Cu") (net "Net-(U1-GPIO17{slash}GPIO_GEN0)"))
 (segment (start 94.9 103.142032) (end 94.9 84.45) (width 0.2) (layer "B.Cu") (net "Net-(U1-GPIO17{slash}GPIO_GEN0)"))
 (segment (start 75.95 97.557717) (end 82.842282 104.45) (width 0.2) (layer "B.Cu") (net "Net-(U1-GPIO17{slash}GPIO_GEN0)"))
 (segment (start 75.95 27.42911) (end 75.95 97.557717) (width 0.2) (layer "B.Cu") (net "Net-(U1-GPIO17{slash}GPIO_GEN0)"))
 (segment (start 82.842282 104.45) (end 93.592032 104.45) (width 0.2) (layer "B.Cu") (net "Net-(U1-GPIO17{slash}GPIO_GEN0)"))
 (segment (start 77.179111 26.2) (end 75.95 27.42911) (width 0.2) (layer "B.Cu") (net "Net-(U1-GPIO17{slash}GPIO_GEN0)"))
 (segment (start 98.650582 26.2) (end 77.179111 26.2) (width 0.2) (layer "B.Cu") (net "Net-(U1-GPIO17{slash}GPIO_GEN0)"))
 (segment (start 100.244 27.793418) (end 98.650582 26.2) (width 0.2) (layer "B.Cu") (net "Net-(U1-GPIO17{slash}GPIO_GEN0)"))
 (segment (start 92.624 31.824) (end 99.626582 31.824) (width 0.2) (layer "B.Cu") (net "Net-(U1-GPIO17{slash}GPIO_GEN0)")))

